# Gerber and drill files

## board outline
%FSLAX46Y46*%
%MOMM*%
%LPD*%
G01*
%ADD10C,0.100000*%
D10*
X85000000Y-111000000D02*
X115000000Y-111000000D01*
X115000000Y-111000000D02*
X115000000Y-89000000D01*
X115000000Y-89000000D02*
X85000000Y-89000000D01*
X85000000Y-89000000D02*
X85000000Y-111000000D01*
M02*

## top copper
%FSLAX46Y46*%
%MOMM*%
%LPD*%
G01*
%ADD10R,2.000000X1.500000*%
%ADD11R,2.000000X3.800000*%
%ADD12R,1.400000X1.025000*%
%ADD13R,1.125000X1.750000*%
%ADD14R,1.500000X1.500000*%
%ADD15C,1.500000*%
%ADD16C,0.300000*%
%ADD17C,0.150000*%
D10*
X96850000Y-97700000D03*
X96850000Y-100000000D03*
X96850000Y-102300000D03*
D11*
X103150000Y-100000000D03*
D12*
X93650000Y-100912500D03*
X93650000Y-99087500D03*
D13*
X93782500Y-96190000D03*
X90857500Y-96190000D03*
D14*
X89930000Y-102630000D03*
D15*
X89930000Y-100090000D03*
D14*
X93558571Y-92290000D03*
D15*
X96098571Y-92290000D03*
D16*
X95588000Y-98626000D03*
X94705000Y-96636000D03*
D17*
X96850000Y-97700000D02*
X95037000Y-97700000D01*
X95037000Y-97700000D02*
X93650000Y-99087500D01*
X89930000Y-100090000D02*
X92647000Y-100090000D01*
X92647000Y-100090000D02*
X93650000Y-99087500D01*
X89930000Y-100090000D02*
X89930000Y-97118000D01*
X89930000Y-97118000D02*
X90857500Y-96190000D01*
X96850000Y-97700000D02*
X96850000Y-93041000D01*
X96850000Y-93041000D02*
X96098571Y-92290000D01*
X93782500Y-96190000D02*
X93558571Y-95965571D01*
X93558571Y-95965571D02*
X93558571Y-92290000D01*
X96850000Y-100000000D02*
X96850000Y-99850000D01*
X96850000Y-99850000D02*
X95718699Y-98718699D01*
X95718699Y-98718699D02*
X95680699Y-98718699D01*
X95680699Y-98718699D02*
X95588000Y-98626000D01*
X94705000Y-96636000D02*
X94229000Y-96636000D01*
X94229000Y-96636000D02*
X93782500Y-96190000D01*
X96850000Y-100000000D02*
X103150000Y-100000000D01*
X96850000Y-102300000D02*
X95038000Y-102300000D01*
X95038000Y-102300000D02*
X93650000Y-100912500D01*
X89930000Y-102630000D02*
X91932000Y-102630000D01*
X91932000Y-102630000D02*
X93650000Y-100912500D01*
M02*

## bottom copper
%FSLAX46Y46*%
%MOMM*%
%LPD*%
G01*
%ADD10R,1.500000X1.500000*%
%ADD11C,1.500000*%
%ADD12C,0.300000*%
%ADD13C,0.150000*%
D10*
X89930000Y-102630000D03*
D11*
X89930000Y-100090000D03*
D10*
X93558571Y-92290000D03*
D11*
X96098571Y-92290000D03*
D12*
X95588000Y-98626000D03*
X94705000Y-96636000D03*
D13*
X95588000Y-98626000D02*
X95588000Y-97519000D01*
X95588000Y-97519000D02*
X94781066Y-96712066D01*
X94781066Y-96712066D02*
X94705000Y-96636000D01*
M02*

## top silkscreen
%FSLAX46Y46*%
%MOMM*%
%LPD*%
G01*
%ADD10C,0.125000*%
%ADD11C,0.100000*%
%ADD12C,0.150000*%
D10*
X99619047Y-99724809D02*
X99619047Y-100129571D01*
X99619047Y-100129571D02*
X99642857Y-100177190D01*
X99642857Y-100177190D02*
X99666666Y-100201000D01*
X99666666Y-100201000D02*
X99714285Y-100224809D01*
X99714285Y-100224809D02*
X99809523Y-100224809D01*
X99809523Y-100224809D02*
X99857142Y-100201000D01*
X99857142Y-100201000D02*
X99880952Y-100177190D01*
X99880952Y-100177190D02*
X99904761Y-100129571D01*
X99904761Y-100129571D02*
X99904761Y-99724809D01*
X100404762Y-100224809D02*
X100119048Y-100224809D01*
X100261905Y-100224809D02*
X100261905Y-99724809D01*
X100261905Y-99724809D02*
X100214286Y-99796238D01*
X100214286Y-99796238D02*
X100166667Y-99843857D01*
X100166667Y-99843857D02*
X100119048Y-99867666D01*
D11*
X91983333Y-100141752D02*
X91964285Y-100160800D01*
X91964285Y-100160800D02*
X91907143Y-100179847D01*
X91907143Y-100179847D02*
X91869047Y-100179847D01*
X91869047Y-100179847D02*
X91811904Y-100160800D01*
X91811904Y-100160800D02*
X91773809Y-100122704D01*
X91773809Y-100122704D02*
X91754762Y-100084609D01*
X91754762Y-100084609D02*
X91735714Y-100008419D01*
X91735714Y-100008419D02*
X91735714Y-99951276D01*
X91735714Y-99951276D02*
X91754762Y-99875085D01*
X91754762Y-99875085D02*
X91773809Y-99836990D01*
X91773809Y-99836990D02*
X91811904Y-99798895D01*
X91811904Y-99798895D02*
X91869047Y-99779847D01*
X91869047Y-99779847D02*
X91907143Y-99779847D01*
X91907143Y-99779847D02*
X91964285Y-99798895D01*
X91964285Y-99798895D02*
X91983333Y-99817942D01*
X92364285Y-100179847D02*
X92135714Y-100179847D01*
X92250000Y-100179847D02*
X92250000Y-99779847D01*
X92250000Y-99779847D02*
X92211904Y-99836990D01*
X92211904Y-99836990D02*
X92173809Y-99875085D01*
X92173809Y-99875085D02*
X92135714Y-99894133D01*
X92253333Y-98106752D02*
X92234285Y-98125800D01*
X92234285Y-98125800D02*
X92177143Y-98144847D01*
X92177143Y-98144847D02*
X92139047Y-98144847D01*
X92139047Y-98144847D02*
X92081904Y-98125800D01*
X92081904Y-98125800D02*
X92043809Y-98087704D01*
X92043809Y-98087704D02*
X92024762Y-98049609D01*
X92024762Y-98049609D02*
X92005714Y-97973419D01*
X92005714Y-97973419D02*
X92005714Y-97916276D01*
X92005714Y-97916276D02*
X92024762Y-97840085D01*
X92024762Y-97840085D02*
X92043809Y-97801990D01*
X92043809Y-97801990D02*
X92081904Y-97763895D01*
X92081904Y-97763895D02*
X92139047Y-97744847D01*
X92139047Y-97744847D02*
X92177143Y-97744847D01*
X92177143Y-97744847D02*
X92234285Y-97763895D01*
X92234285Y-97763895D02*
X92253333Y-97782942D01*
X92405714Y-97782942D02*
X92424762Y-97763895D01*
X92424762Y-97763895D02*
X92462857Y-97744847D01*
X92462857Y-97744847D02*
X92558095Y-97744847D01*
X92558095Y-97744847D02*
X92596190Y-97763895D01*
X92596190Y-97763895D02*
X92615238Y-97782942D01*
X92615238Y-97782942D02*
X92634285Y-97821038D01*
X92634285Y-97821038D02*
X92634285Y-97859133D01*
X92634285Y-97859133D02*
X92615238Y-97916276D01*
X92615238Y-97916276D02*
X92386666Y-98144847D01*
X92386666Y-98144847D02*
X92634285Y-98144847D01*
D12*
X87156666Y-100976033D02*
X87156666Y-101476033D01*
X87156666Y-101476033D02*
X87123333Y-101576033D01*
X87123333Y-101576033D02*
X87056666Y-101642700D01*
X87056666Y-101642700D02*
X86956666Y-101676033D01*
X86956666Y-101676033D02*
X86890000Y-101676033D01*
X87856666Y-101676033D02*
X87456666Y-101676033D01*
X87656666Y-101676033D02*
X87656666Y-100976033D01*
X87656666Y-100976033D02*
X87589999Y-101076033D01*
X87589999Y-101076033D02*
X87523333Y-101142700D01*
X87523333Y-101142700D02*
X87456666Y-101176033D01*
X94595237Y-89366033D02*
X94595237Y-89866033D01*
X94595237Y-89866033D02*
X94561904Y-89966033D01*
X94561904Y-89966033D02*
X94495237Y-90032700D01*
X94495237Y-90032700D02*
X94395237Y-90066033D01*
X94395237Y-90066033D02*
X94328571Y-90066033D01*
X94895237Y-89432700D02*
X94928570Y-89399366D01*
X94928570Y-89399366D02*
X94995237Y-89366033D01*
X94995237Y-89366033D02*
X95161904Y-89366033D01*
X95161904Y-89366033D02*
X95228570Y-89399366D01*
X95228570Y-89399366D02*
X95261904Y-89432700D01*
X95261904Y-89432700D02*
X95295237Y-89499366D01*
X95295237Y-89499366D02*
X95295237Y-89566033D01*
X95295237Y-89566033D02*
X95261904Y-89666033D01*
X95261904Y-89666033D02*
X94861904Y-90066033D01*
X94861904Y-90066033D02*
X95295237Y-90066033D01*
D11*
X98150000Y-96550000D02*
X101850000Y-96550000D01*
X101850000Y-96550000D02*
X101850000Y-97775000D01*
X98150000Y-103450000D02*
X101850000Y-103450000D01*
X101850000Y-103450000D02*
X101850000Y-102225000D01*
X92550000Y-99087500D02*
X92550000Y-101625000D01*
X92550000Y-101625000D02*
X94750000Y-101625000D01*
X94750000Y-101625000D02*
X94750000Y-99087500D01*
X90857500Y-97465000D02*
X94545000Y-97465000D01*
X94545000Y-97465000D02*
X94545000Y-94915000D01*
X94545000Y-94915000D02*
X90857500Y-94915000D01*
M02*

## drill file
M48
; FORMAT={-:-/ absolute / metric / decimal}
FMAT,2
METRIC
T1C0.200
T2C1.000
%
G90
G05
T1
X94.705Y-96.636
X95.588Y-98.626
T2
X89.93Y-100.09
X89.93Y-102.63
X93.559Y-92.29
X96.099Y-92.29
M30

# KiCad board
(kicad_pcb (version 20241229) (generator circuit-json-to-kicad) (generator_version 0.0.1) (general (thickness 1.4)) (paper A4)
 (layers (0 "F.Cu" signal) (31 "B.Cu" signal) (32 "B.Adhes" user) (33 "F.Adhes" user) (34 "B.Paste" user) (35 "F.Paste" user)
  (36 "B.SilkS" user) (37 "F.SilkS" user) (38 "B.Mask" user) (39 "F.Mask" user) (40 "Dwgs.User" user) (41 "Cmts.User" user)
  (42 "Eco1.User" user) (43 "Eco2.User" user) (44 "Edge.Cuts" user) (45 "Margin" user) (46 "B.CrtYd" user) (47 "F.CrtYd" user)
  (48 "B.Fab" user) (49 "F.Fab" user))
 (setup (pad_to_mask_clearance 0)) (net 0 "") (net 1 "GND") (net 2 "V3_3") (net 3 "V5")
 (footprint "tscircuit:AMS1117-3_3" (layer F.Cu) (at 100 100 0)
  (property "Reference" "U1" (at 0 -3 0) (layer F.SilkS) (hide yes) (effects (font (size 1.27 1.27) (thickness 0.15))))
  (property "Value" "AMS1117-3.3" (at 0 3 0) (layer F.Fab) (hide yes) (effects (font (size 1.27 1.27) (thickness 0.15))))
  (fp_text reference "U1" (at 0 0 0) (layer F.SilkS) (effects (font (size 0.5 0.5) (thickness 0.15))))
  (fp_line (start -1.85 -3.45) (end 1.85 -3.45) (stroke (width 0.1) (type default)) (layer F.SilkS))
  (fp_line (start 1.85 -3.45) (end 1.85 -2.225) (stroke (width 0.1) (type default)) (layer F.SilkS))
  (fp_line (start -1.85 3.45) (end 1.85 3.45) (stroke (width 0.1) (type default)) (layer F.SilkS))
  (fp_line (start 1.85 3.45) (end 1.85 2.225) (stroke (width 0.1) (type default)) (layer F.SilkS))
  (pad "1" smd rect (at -3.15 -2.3 0) (size 2 1.5) (layers F.Cu F.Paste F.Mask) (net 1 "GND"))
  (pad "2" smd rect (at -3.15 0 0) (size 2 1.5) (layers F.Cu F.Paste F.Mask) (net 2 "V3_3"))
  (pad "3" smd rect (at -3.15 2.3 0) (size 2 1.5) (layers F.Cu F.Paste F.Mask) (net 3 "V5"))
  (pad "4" smd rect (at 3.15 0 0) (size 2 3.8) (layers F.Cu F.Paste F.Mask) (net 2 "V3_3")))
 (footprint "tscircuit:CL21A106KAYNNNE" (layer F.Cu) (at 93.65 100 90)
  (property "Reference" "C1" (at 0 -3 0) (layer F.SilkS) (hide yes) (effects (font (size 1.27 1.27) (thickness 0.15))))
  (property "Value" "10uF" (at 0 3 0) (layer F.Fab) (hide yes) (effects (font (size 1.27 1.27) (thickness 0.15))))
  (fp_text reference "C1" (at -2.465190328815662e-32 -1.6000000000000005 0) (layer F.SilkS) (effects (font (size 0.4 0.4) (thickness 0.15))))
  (fp_line (start 0.9125 -1.1000000000000005) (end -1.6249999999999998 -1.1000000000000005) (stroke (width 0.1) (type default))
   (layer F.SilkS))
  (fp_line (start -1.6249999999999998 -1.1000000000000005) (end -1.6249999999999998 1.1000000000000005) (stroke (width 0.1) (type default))
   (layer F.SilkS))
  (fp_line (start -1.6249999999999998 1.1000000000000005) (end 0.9125 1.1000000000000005) (stroke (width 0.1) (type default))
   (layer F.SilkS))
  (pad "1" smd rect (at -0.9125 0 0) (size 1.4 1.025) (layers F.Cu F.Paste F.Mask) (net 3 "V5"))
  (pad "2" smd rect (at 0.9125 0 0) (size 1.4 1.025) (layers F.Cu F.Paste F.Mask) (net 1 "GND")))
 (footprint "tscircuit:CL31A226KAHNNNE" (layer F.Cu) (at 92.32 96.19 180)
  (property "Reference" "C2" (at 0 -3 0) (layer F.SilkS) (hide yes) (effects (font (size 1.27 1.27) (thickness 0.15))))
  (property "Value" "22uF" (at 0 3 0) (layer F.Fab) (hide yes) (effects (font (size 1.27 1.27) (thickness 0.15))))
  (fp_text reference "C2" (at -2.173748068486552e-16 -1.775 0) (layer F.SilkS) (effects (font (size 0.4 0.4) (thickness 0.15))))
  (fp_line (start 1.4625000000000001 -1.2749999999999997) (end -2.2249999999999996 -1.2750000000000001) (stroke (width 0.1) (type default))
   (layer F.SilkS))
  (fp_line (start -2.2249999999999996 -1.2750000000000001) (end -2.2249999999999996 1.2749999999999997) (stroke (width 0.1) (type default))
   (layer F.SilkS))
  (fp_line (start -2.2249999999999996 1.2749999999999997) (end 1.4625000000000006 1.2750000000000001) (stroke (width 0.1) (type default))
   (layer F.SilkS))
  (pad "1" smd rect (at -1.4625000000000004 0 0) (size 1.125 1.75) (layers F.Cu F.Paste F.Mask) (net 2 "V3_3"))
  (pad "2" smd rect (at 1.4624999999999995 -4.440892098500626e-16 0) (size 1.125 1.75) (layers F.Cu F.Paste F.Mask) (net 1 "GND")))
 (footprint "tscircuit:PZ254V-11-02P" (layer F.Cu) (at 89.93 101.36 90)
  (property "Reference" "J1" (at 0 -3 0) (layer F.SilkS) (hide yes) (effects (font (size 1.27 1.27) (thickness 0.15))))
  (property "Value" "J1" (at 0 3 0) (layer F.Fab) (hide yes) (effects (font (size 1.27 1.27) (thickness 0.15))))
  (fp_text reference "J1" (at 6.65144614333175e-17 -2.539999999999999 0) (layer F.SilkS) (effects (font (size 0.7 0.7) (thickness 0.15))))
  (pad "1" thru_hole rect (at -1.27 7.776507174585693e-17 0) (size 1.5 1.5) (drill 1) (layers *.Cu *.Mask) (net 3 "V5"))
  (pad "2" thru_hole circle (at 1.27 -7.776507174585693e-17 0) (size 1.5 1.5) (drill 1) (layers *.Cu *.Mask) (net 1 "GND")))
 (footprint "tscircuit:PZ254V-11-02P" (layer F.Cu) (at 94.82857142857142 92.29 0)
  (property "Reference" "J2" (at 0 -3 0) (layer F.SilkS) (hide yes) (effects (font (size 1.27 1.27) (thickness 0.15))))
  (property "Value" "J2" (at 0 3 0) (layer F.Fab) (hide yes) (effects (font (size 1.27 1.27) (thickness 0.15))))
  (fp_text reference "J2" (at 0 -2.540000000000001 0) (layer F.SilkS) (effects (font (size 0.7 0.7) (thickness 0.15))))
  (pad "1" thru_hole rect (at -1.2699999999999996 0 0) (size 1.5 1.5) (drill 1) (layers *.Cu *.Mask) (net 2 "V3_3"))
  (pad "2" thru_hole circle (at 1.27 0 0) (size 1.5 1.5) (drill 1) (layers *.Cu *.Mask) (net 1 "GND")))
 (segment (start 96.85 97.7) (end 95.037 97.7) (width 0.15) (layer F.Cu) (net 1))
 (segment (start 95.037 97.7) (end 93.65 99.0875) (width 0.15) (layer F.Cu) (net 1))
 (segment (start 89.93 100.09) (end 92.647 100.09) (width 0.15) (layer F.Cu) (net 1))
 (segment (start 92.647 100.09) (end 93.65 99.0875) (width 0.15) (layer F.Cu) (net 1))
 (segment (start 89.93 100.09) (end 89.93 97.118) (width 0.15) (layer F.Cu) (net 1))
 (segment (start 89.93 97.118) (end 90.8575 96.19) (width 0.15) (layer F.Cu) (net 1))
 (segment (start 96.85 97.7) (end 96.85 93.041) (width 0.15) (layer F.Cu) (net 1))
 (segment (start 96.85 93.041) (end 96.09857142857143 92.29) (width 0.15) (layer F.Cu) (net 1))
 (segment (start 93.7825 96.19) (end 93.55857142857143 95.96557142857142) (width 0.15) (layer F.Cu) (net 2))
 (segment (start 93.55857142857143 95.96557142857142) (end 93.55857142857143 92.29) (width 0.15) (layer F.Cu) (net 2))
 (segment (start 96.85 100) (end 96.85 99.85) (width 0.15) (layer F.Cu) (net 2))
 (segment (start 96.85 99.85) (end 95.71869926606536 98.71869926606536) (width 0.15) (layer F.Cu) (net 2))
 (segment (start 95.71869926606536 98.71869926606536) (end 95.68069926606536 98.71869926606536) (width 0.15) (layer F.Cu) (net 2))
 (segment (start 95.68069926606536 98.71869926606536) (end 95.588 98.626) (width 0.15) (layer F.Cu) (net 2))
 (segment (start 95.588 98.626) (end 95.588 97.519) (width 0.15) (layer B.Cu) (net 2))
 (segment (start 95.588 97.519) (end 94.78106563670283 96.71206563670283) (width 0.15) (layer B.Cu) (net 2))
 (segment (start 94.78106563670283 96.71206563670283) (end 94.705 96.636) (width 0.15) (layer B.Cu) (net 2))
 (segment (start 94.705 96.636) (end 94.229 96.636) (width 0.15) (layer F.Cu) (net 2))
 (segment (start 94.229 96.636) (end 93.7825 96.19) (width 0.15) (layer F.Cu) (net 2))
 (segment (start 96.85 100) (end 103.15 100) (width 0.15) (layer F.Cu) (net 2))
 (segment (start 96.85 102.3) (end 95.038 102.3) (width 0.15) (layer F.Cu) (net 3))
 (segment (start 95.038 102.3) (end 93.65 100.9125) (width 0.15) (layer F.Cu) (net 3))
 (segment (start 89.93 102.63) (end 91.932 102.63) (width 0.15) (layer F.Cu) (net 3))
 (segment (start 91.932 102.63) (end 93.65 100.9125) (width 0.15) (layer F.Cu) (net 3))
 (gr_line (start 85 111) (end 115 111) (width 0.1) (layer Edge.Cuts))
 (gr_line (start 115 111) (end 115 89) (width 0.1) (layer Edge.Cuts))
 (gr_line (start 115 89) (end 85 89) (width 0.1) (layer Edge.Cuts))
 (gr_line (start 85 89) (end 85 111) (width 0.1) (layer Edge.Cuts))
 (via (at 95.588 98.626) (size 0.3) (drill 0.2) (layers F.Cu B.Cu) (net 2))
 (via (at 94.705 96.636) (size 0.3) (drill 0.2) (layers F.Cu B.Cu) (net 2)))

